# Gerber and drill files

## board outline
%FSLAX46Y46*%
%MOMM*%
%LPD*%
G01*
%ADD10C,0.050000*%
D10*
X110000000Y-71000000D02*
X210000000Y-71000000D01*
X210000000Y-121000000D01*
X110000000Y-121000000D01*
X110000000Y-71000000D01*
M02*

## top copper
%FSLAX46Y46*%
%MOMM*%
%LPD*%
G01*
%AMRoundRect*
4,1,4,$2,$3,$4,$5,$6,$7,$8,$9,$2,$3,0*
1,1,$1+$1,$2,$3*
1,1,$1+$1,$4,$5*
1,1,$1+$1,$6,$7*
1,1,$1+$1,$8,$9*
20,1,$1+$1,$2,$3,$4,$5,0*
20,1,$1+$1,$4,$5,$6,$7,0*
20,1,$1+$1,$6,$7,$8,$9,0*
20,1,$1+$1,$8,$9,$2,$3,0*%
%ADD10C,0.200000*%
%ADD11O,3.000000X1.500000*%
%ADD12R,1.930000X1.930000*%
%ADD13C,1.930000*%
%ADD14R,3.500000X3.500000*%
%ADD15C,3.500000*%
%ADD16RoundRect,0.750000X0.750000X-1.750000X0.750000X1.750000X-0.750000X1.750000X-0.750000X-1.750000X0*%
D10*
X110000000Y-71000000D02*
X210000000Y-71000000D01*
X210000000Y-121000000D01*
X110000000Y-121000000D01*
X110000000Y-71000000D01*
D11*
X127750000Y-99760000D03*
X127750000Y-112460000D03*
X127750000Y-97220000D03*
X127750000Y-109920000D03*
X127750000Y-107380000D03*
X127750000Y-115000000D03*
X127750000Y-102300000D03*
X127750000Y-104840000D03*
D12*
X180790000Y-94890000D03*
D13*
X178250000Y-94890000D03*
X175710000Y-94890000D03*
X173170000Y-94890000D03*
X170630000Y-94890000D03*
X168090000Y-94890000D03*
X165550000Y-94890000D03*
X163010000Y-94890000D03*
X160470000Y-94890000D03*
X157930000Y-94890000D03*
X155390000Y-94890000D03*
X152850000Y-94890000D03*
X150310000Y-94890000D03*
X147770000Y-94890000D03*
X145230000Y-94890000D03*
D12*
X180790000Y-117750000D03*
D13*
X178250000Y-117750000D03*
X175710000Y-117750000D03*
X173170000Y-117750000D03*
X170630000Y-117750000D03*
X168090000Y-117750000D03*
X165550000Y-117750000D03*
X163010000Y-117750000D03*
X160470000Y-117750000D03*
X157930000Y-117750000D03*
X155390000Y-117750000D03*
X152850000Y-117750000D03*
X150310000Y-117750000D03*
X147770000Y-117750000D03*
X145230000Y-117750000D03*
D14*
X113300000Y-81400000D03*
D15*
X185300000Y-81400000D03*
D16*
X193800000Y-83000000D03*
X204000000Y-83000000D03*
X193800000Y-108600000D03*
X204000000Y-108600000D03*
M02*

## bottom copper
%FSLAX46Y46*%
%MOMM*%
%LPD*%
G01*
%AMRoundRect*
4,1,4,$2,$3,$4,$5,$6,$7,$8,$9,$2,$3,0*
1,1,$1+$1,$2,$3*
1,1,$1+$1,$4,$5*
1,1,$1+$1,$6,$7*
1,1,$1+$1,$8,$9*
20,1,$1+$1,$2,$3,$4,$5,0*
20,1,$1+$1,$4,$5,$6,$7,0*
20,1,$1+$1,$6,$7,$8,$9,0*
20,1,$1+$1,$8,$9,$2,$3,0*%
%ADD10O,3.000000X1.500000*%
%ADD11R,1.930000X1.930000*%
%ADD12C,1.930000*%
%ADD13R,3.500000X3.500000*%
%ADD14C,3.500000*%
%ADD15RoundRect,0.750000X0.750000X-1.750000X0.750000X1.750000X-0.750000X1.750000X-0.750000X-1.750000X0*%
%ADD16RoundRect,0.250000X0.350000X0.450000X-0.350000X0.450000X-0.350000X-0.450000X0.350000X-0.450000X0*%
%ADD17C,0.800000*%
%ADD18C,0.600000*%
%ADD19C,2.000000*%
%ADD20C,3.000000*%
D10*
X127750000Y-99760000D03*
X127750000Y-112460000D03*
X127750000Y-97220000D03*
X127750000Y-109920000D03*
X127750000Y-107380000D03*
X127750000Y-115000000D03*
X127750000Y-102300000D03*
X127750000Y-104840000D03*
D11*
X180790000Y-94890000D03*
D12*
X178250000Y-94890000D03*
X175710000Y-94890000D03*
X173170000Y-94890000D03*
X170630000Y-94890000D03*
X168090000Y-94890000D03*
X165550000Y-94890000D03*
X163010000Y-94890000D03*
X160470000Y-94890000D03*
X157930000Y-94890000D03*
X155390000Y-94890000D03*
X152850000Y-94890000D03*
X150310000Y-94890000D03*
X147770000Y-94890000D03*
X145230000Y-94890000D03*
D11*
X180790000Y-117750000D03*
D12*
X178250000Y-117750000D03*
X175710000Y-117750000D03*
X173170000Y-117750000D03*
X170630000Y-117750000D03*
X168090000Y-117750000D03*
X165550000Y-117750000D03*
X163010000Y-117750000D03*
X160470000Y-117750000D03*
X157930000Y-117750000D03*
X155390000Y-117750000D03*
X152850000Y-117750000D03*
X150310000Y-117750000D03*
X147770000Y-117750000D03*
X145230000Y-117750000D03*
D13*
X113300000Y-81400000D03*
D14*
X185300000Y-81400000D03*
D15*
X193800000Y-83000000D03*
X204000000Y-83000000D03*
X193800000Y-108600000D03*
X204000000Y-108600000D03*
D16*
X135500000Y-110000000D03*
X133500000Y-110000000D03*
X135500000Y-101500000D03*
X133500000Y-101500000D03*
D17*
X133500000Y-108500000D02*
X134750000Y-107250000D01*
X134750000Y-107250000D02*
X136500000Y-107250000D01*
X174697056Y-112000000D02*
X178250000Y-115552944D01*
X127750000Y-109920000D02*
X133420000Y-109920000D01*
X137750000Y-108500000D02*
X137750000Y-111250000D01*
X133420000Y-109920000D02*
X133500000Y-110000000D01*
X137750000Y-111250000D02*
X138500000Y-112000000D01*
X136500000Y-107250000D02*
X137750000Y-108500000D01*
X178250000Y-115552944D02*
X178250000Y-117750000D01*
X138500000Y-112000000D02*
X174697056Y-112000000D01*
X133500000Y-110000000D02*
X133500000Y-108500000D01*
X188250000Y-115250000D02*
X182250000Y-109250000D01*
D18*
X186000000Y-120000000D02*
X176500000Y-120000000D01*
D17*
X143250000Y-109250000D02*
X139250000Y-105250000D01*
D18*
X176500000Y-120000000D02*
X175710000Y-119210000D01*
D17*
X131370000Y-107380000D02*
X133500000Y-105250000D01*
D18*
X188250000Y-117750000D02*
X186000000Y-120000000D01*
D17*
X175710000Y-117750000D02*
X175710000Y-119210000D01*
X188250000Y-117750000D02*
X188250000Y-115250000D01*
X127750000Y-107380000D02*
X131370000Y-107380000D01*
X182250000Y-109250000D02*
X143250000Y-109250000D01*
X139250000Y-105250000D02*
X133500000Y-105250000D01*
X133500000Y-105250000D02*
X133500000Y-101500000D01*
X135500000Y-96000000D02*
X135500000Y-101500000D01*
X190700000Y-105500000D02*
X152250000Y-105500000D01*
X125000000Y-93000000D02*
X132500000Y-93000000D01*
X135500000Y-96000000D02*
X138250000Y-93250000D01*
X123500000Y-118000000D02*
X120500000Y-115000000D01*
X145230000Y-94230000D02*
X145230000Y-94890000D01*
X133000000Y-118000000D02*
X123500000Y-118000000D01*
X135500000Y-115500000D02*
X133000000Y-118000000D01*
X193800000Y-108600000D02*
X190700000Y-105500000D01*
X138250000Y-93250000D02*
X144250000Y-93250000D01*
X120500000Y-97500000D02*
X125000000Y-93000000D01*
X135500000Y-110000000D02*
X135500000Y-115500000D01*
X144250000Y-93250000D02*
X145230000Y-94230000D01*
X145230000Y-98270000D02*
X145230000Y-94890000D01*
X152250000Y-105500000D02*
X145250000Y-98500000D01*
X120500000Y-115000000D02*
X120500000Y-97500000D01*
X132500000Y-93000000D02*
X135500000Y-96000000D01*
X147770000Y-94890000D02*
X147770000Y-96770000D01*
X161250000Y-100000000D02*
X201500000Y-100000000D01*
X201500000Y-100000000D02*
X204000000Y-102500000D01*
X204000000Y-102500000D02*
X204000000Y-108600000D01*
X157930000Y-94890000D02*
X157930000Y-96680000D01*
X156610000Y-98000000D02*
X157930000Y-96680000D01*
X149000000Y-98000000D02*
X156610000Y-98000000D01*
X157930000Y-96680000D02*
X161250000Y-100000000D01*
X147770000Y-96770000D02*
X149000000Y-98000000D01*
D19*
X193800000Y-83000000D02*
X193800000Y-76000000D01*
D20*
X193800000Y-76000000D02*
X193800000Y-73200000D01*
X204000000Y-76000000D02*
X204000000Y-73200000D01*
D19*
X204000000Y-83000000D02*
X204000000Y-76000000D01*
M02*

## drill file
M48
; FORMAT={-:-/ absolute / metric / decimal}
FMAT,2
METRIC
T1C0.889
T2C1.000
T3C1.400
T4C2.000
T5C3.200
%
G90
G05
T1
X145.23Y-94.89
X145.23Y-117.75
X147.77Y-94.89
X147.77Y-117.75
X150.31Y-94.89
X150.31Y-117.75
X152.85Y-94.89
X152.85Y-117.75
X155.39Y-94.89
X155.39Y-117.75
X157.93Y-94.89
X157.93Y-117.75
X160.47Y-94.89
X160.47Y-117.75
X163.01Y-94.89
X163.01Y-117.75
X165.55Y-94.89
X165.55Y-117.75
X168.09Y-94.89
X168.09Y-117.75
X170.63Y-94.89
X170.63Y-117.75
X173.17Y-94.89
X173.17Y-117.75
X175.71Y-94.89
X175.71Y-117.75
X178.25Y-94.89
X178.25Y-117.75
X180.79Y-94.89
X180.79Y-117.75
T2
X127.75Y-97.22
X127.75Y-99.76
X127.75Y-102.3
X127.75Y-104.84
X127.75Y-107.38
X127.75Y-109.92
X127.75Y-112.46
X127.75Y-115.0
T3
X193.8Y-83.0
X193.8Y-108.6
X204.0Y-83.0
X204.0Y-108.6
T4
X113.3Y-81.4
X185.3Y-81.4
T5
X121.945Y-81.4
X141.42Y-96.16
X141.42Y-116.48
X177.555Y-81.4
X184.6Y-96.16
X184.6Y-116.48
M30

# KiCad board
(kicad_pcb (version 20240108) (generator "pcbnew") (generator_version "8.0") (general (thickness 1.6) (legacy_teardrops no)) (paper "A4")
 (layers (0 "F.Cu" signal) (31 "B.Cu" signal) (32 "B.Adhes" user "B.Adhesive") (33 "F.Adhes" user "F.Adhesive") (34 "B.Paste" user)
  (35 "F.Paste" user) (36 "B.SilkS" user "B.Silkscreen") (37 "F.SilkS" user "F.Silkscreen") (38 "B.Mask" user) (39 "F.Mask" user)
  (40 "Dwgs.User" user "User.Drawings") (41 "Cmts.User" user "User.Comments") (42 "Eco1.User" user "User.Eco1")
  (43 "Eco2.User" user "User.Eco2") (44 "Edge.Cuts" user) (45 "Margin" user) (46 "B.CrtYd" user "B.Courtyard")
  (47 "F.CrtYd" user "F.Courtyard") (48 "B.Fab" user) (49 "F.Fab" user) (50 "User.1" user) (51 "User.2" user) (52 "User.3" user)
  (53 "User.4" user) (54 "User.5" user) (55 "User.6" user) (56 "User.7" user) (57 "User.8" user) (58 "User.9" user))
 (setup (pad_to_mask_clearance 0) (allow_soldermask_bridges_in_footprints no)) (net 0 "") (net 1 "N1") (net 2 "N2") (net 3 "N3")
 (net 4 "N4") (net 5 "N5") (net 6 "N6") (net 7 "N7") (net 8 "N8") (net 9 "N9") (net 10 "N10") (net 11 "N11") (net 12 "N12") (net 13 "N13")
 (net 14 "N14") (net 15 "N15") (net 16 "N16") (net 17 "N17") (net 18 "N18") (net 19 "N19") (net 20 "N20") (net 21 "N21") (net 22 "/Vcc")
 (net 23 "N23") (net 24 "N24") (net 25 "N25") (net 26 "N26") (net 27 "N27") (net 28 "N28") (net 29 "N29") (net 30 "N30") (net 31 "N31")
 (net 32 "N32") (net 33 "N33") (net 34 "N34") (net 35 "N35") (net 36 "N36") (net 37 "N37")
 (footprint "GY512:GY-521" (layer "F.Cu") (at 129.52 95.156 180)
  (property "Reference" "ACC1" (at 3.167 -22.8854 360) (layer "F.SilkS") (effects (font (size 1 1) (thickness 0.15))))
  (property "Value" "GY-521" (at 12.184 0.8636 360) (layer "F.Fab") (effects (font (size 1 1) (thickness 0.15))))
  (pad "AD0" thru_hole oval (at 1.77 -4.604 180) (size 3 1.5) (drill 1) (layers "*.Cu" "*.Mask") (remove_unused_layers no) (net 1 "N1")
   (solder_mask_margin 0.102))
  (pad "GND" thru_hole oval (at 1.77 -17.304 180) (size 3 1.5) (drill 1) (layers "*.Cu" "*.Mask") (remove_unused_layers no) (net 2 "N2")
   (solder_mask_margin 0.102))
  (pad "INT" thru_hole oval (at 1.77 -2.064 180) (size 3 1.5) (drill 1) (layers "*.Cu" "*.Mask") (remove_unused_layers no) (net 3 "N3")
   (solder_mask_margin 0.102))
  (pad "SCL" thru_hole oval (at 1.77 -14.764 180) (size 3 1.5) (drill 1) (layers "*.Cu" "*.Mask") (remove_unused_layers no) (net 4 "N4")
   (solder_mask_margin 0.102))
  (pad "SDA" thru_hole oval (at 1.77 -12.224 180) (size 3 1.5) (drill 1) (layers "*.Cu" "*.Mask") (remove_unused_layers no) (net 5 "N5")
   (solder_mask_margin 0.102))
  (pad "VCC" thru_hole oval (at 1.77 -19.844 180) (size 3 1.5) (drill 1) (layers "*.Cu" "*.Mask") (remove_unused_layers no) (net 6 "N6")
   (solder_mask_margin 0.102))
  (pad "XCL" thru_hole oval (at 1.77 -7.144 180) (size 3 1.5) (drill 1) (layers "*.Cu" "*.Mask") (remove_unused_layers no) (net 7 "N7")
   (solder_mask_margin 0.102))
  (pad "XDA" thru_hole oval (at 1.77 -9.684 180) (size 3 1.5) (drill 1) (layers "*.Cu" "*.Mask") (remove_unused_layers no) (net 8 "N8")
   (solder_mask_margin 0.102)))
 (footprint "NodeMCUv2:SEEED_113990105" (layer "F.Cu") (at 163.01 106.32 -90)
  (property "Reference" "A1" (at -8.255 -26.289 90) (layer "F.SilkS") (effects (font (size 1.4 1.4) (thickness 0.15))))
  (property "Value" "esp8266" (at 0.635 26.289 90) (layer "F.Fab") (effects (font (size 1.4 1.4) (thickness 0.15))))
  (pad "" np_thru_hole circle (at -10.16 -21.59 270) (size 3.2 3.2) (drill 3.2) (layers "*.Cu" "*.Mask"))
  (pad "" np_thru_hole circle (at -10.16 21.59 270) (size 3.2 3.2) (drill 3.2) (layers "*.Cu" "*.Mask"))
  (pad "" np_thru_hole circle (at 10.16 -21.59 270) (size 3.2 3.2) (drill 3.2) (layers "*.Cu" "*.Mask"))
  (pad "" np_thru_hole circle (at 10.16 21.59 270) (size 3.2 3.2) (drill 3.2) (layers "*.Cu" "*.Mask"))
  (pad "J1_1" thru_hole rect (at -11.43 -17.78 270) (size 1.93 1.93) (drill 0.889) (layers "*.Cu" "*.Mask") (remove_unused_layers no)
   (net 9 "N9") (solder_mask_margin 0.102))
  (pad "J1_2" thru_hole circle (at -11.43 -15.24 270) (size 1.93 1.93) (drill 0.889) (layers "*.Cu" "*.Mask") (remove_unused_layers no)
   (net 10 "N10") (solder_mask_margin 0.102))
  (pad "J1_3" thru_hole circle (at -11.43 -12.7 270) (size 1.93 1.93) (drill 0.889) (layers "*.Cu" "*.Mask") (remove_unused_layers no)
   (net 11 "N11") (solder_mask_margin 0.102))
  (pad "J1_4" thru_hole circle (at -11.43 -10.16 270) (size 1.93 1.93) (drill 0.889) (layers "*.Cu" "*.Mask") (remove_unused_layers no)
   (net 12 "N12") (solder_mask_margin 0.102))
  (pad "J1_5" thru_hole circle (at -11.43 -7.62 270) (size 1.93 1.93) (drill 0.889) (layers "*.Cu" "*.Mask") (remove_unused_layers no)
   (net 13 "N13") (solder_mask_margin 0.102))
  (pad "J1_6" thru_hole circle (at -11.43 -5.08 270) (size 1.93 1.93) (drill 0.889) (layers "*.Cu" "*.Mask") (remove_unused_layers no)
   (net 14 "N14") (solder_mask_margin 0.102))
  (pad "J1_7" thru_hole circle (at -11.43 -2.54 270) (size 1.93 1.93) (drill 0.889) (layers "*.Cu" "*.Mask") (remove_unused_layers no)
   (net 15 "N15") (solder_mask_margin 0.102))
  (pad "J1_8" thru_hole circle (at -11.43 0 270) (size 1.93 1.93) (drill 0.889) (layers "*.Cu" "*.Mask") (remove_unused_layers no)
   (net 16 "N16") (solder_mask_margin 0.102))
  (pad "J1_9" thru_hole circle (at -11.43 2.54 270) (size 1.93 1.93) (drill 0.889) (layers "*.Cu" "*.Mask") (remove_unused_layers no)
   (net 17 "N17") (solder_mask_margin 0.102))
  (pad "J1_10" thru_hole circle (at -11.43 5.08 270) (size 1.93 1.93) (drill 0.889) (layers "*.Cu" "*.Mask") (remove_unused_layers no)
   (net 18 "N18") (solder_mask_margin 0.102))
  (pad "J1_11" thru_hole circle (at -11.43 7.62 270) (size 1.93 1.93) (drill 0.889) (layers "*.Cu" "*.Mask") (remove_unused_layers no)
   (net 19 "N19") (solder_mask_margin 0.102))
  (pad "J1_12" thru_hole circle (at -11.43 10.16 270) (size 1.93 1.93) (drill 0.889) (layers "*.Cu" "*.Mask") (remove_unused_layers no)
   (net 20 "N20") (solder_mask_margin 0.102))
  (pad "J1_13" thru_hole circle (at -11.43 12.7 270) (size 1.93 1.93) (drill 0.889) (layers "*.Cu" "*.Mask") (remove_unused_layers no)
   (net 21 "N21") (solder_mask_margin 0.102))
  (pad "J1_14" thru_hole circle (at -11.43 15.24 270) (size 1.93 1.93) (drill 0.889) (layers "*.Cu" "*.Mask") (remove_unused_layers no)
   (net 18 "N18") (solder_mask_margin 0.102))
  (pad "J1_15" thru_hole circle (at -11.43 17.78 270) (size 1.93 1.93) (drill 0.889) (layers "*.Cu" "*.Mask") (remove_unused_layers no)
   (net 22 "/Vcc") (solder_mask_margin 0.102))
  (pad "J2_1" thru_hole rect (at 11.43 -17.78 270) (size 1.93 1.93) (drill 0.889) (layers "*.Cu" "*.Mask") (remove_unused_layers no)
   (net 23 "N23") (solder_mask_margin 0.102))
  (pad "J2_2" thru_hole circle (at 11.43 -15.24 270) (size 1.93 1.93) (drill 0.889) (layers "*.Cu" "*.Mask") (remove_unused_layers no)
   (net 4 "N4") (solder_mask_margin 0.102))
  (pad "J2_3" thru_hole circle (at 11.43 -12.7 270) (size 1.93 1.93) (drill 0.889) (layers "*.Cu" "*.Mask") (remove_unused_layers no)
   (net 5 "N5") (solder_mask_margin 0.102))
  (pad "J2_4" thru_hole circle (at 11.43 -10.16 270) (size 1.93 1.93) (drill 0.889) (layers "*.Cu" "*.Mask") (remove_unused_layers no)
   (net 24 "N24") (solder_mask_margin 0.102))
  (pad "J2_5" thru_hole circle (at 11.43 -7.62 270) (size 1.93 1.93) (drill 0.889) (layers "*.Cu" "*.Mask") (remove_unused_layers no)
   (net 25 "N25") (solder_mask_margin 0.102))
  (pad "J2_6" thru_hole circle (at 11.43 -5.08 270) (size 1.93 1.93) (drill 0.889) (layers "*.Cu" "*.Mask") (remove_unused_layers no)
   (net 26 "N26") (solder_mask_margin 0.102))
  (pad "J2_7" thru_hole circle (at 11.43 -2.54 270) (size 1.93 1.93) (drill 0.889) (layers "*.Cu" "*.Mask") (remove_unused_layers no)
   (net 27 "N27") (solder_mask_margin 0.102))
  (pad "J2_8" thru_hole circle (at 11.43 0 270) (size 1.93 1.93) (drill 0.889) (layers "*.Cu" "*.Mask") (remove_unused_layers no)
   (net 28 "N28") (solder_mask_margin 0.102))
  (pad "J2_9" thru_hole circle (at 11.43 2.54 270) (size 1.93 1.93) (drill 0.889) (layers "*.Cu" "*.Mask") (remove_unused_layers no)
   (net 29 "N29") (solder_mask_margin 0.102))
  (pad "J2_10" thru_hole circle (at 11.43 5.08 270) (size 1.93 1.93) (drill 0.889) (layers "*.Cu" "*.Mask") (remove_unused_layers no)
   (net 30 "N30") (solder_mask_margin 0.102))
  (pad "J2_11" thru_hole circle (at 11.43 7.62 270) (size 1.93 1.93) (drill 0.889) (layers "*.Cu" "*.Mask") (remove_unused_layers no)
   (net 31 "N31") (solder_mask_margin 0.102))
  (pad "J2_12" thru_hole circle (at 11.43 10.16 270) (size 1.93 1.93) (drill 0.889) (layers "*.Cu" "*.Mask") (remove_unused_layers no)
   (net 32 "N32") (solder_mask_margin 0.102))
  (pad "J2_13" thru_hole circle (at 11.43 12.7 270) (size 1.93 1.93) (drill 0.889) (layers "*.Cu" "*.Mask") (remove_unused_layers no)
   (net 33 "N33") (solder_mask_margin 0.102))
  (pad "J2_14" thru_hole circle (at 11.43 15.24 270) (size 1.93 1.93) (drill 0.889) (layers "*.Cu" "*.Mask") (remove_unused_layers no)
   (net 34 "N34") (solder_mask_margin 0.102))
  (pad "J2_15" thru_hole circle (at 11.43 17.78 270) (size 1.93 1.93) (drill 0.889) (layers "*.Cu" "*.Mask") (remove_unused_layers no)
   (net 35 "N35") (solder_mask_margin 0.102)))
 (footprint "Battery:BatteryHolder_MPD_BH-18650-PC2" (layer "F.Cu") (at 113.3 81.4)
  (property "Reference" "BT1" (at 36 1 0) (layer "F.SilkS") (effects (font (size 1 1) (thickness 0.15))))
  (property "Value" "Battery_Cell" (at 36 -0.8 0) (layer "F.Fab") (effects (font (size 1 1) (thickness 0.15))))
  (pad "" np_thru_hole circle (at 8.645 0) (size 3.2 3.2) (drill 3.2) (layers "*.Cu" "*.Mask"))
  (pad "" np_thru_hole circle (at 64.255 0) (size 3.2 3.2) (drill 3.2) (layers "*.Cu" "*.Mask"))
  (pad "1" thru_hole rect (at 0 0) (size 3.5 3.5) (drill 2) (layers "*.Cu" "*.Mask") (remove_unused_layers no) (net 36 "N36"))
  (pad "2" thru_hole circle (at 72 0) (size 3.5 3.5) (drill 2) (layers "*.Cu" "*.Mask") (remove_unused_layers no) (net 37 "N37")))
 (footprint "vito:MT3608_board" (layer "F.Cu") (at 207.4 114.3 90)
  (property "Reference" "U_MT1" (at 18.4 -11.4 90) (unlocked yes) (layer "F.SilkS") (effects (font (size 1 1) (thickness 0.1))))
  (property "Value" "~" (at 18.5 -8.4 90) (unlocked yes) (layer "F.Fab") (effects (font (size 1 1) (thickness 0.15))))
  (pad "1" thru_hole roundrect (at 31.3 -13.6 90) (size 5 3) (drill 1.4) (layers "*.Cu" "*.Mask") (remove_unused_layers no)
   (roundrect_rratio 0.25) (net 36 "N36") (thermal_bridge_angle 45))
  (pad "2" thru_hole roundrect (at 31.3 -3.4 90) (size 5 3) (drill 1.4) (layers "*.Cu" "*.Mask") (remove_unused_layers no)
   (roundrect_rratio 0.25) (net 37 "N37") (thermal_bridge_angle 45))
  (pad "3" thru_hole roundrect (at 5.7 -13.6 90) (size 5 3) (drill 1.4) (layers "*.Cu" "*.Mask") (remove_unused_layers no)
   (roundrect_rratio 0.25) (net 22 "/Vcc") (thermal_bridge_angle 45))
  (pad "4" thru_hole roundrect (at 5.7 -3.4 90) (size 5 3) (drill 1.4) (layers "*.Cu" "*.Mask") (remove_unused_layers no)
   (roundrect_rratio 0.25) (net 18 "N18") (thermal_bridge_angle 45)))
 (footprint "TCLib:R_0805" (layer "B.Cu") (at 134.5 110 180)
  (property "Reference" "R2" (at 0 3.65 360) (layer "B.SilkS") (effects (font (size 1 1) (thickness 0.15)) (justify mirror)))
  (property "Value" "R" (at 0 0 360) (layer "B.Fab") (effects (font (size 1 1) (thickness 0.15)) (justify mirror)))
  (pad "1" smd roundrect (at -1 0 180) (size 1.2 1.4) (layers "B.Cu" "B.Paste" "B.Mask") (roundrect_rratio 0.208333) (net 22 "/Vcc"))
  (pad "2" smd roundrect (at 1 0 180) (size 1.2 1.4) (layers "B.Cu" "B.Paste" "B.Mask") (roundrect_rratio 0.208333) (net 4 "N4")))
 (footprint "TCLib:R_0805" (layer "B.Cu") (at 134.5 101.5 180)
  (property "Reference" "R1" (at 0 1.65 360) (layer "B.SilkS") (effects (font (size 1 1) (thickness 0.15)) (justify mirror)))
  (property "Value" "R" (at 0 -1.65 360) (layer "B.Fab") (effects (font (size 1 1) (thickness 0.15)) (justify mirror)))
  (pad "1" smd roundrect (at -1 0 180) (size 1.2 1.4) (layers "B.Cu" "B.Paste" "B.Mask") (roundrect_rratio 0.208333) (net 22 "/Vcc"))
  (pad "2" smd roundrect (at 1 0 180) (size 1.2 1.4) (layers "B.Cu" "B.Paste" "B.Mask") (roundrect_rratio 0.208333) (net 5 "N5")))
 (gr_rect (start 110 71) (end 210 121) (stroke (width 0.2) (type default)) (fill none) (layer "F.Cu") (net 4))
 (gr_rect (start 110 71) (end 210 121) (stroke (width 0.05) (type default)) (fill none) (layer "Edge.Cuts"))
 (segment (start 133.5 108.5) (end 134.75 107.25) (width 0.8) (layer "B.Cu") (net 4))
 (segment (start 134.75 107.25) (end 136.5 107.25) (width 0.8) (layer "B.Cu") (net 4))
 (segment (start 174.697056 112) (end 178.25 115.552944) (width 0.8) (layer "B.Cu") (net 4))
 (segment (start 127.75 109.92) (end 133.42 109.92) (width 0.8) (layer "B.Cu") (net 4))
 (segment (start 137.75 108.5) (end 137.75 111.25) (width 0.8) (layer "B.Cu") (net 4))
 (segment (start 133.42 109.92) (end 133.5 110) (width 0.8) (layer "B.Cu") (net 4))
 (segment (start 137.75 111.25) (end 138.5 112) (width 0.8) (layer "B.Cu") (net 4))
 (segment (start 136.5 107.25) (end 137.75 108.5) (width 0.8) (layer "B.Cu") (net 4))
 (segment (start 178.25 115.552944) (end 178.25 117.75) (width 0.8) (layer "B.Cu") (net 4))
 (segment (start 138.5 112) (end 174.697056 112) (width 0.8) (layer "B.Cu") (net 4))
 (segment (start 133.5 110) (end 133.5 108.5) (width 0.8) (layer "B.Cu") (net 4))
 (segment (start 188.25 115.25) (end 182.25 109.25) (width 0.8) (layer "B.Cu") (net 5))
 (segment (start 186 120) (end 176.5 120) (width 0.6) (layer "B.Cu") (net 5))
 (segment (start 143.25 109.25) (end 139.25 105.25) (width 0.8) (layer "B.Cu") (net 5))
 (segment (start 176.5 120) (end 175.71 119.21) (width 0.6) (layer "B.Cu") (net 5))
 (segment (start 131.37 107.38) (end 133.5 105.25) (width 0.8) (layer "B.Cu") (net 5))
 (segment (start 188.25 117.75) (end 186 120) (width 0.6) (layer "B.Cu") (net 5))
 (segment (start 175.71 117.75) (end 175.71 119.21) (width 0.8) (layer "B.Cu") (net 5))
 (segment (start 188.25 117.75) (end 188.25 115.25) (width 0.8) (layer "B.Cu") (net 5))
 (segment (start 127.75 107.38) (end 131.37 107.38) (width 0.8) (layer "B.Cu") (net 5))
 (segment (start 182.25 109.25) (end 143.25 109.25) (width 0.8) (layer "B.Cu") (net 5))
 (segment (start 139.25 105.25) (end 133.5 105.25) (width 0.8) (layer "B.Cu") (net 5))
 (segment (start 133.5 105.25) (end 133.5 101.5) (width 0.8) (layer "B.Cu") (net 5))
 (segment (start 135.5 96) (end 135.5 101.5) (width 0.8) (layer "B.Cu") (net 22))
 (segment (start 190.7 105.5) (end 152.25 105.5) (width 0.8) (layer "B.Cu") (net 22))
 (segment (start 125 93) (end 132.5 93) (width 0.8) (layer "B.Cu") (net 22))
 (segment (start 135.5 96) (end 138.25 93.25) (width 0.8) (layer "B.Cu") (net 22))
 (segment (start 123.5 118) (end 120.5 115) (width 0.8) (layer "B.Cu") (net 22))
 (segment (start 145.23 94.23) (end 145.23 94.89) (width 0.8) (layer "B.Cu") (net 22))
 (segment (start 133 118) (end 123.5 118) (width 0.8) (layer "B.Cu") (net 22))
 (segment (start 135.5 115.5) (end 133 118) (width 0.8) (layer "B.Cu") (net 22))
 (segment (start 193.8 108.6) (end 190.7 105.5) (width 0.8) (layer "B.Cu") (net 22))
 (segment (start 138.25 93.25) (end 144.25 93.25) (width 0.8) (layer "B.Cu") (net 22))
 (segment (start 120.5 97.5) (end 125 93) (width 0.8) (layer "B.Cu") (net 22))
 (segment (start 135.5 110) (end 135.5 115.5) (width 0.8) (layer "B.Cu") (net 22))
 (segment (start 144.25 93.25) (end 145.23 94.23) (width 0.8) (layer "B.Cu") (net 22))
 (segment (start 145.23 98.27) (end 145.23 94.89) (width 0.8) (layer "B.Cu") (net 22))
 (segment (start 152.25 105.5) (end 145.25 98.5) (width 0.8) (layer "B.Cu") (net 22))
 (segment (start 120.5 115) (end 120.5 97.5) (width 0.8) (layer "B.Cu") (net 22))
 (segment (start 132.5 93) (end 135.5 96) (width 0.8) (layer "B.Cu") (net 22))
 (segment (start 147.77 94.89) (end 147.77 96.77) (width 0.8) (layer "B.Cu") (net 18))
 (segment (start 161.25 100) (end 201.5 100) (width 0.8) (layer "B.Cu") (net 18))
 (segment (start 201.5 100) (end 204 102.5) (width 0.8) (layer "B.Cu") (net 18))
 (segment (start 204 102.5) (end 204 108.6) (width 0.8) (layer "B.Cu") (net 18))
 (segment (start 157.93 94.89) (end 157.93 96.68) (width 0.8) (layer "B.Cu") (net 18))
 (segment (start 156.61 98) (end 157.93 96.68) (width 0.8) (layer "B.Cu") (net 18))
 (segment (start 149 98) (end 156.61 98) (width 0.8) (layer "B.Cu") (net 18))
 (segment (start 157.93 96.68) (end 161.25 100) (width 0.8) (layer "B.Cu") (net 18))
 (segment (start 147.77 96.77) (end 149 98) (width 0.8) (layer "B.Cu") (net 18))
 (segment (start 193.8 83) (end 193.8 76) (width 2) (layer "B.Cu") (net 36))
 (segment (start 193.8 76) (end 193.8 73.2) (width 3) (layer "B.Cu") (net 36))
 (segment (start 204 76) (end 204 73.2) (width 3) (layer "B.Cu") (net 37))
 (segment (start 204 83) (end 204 76) (width 2) (layer "B.Cu") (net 37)))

